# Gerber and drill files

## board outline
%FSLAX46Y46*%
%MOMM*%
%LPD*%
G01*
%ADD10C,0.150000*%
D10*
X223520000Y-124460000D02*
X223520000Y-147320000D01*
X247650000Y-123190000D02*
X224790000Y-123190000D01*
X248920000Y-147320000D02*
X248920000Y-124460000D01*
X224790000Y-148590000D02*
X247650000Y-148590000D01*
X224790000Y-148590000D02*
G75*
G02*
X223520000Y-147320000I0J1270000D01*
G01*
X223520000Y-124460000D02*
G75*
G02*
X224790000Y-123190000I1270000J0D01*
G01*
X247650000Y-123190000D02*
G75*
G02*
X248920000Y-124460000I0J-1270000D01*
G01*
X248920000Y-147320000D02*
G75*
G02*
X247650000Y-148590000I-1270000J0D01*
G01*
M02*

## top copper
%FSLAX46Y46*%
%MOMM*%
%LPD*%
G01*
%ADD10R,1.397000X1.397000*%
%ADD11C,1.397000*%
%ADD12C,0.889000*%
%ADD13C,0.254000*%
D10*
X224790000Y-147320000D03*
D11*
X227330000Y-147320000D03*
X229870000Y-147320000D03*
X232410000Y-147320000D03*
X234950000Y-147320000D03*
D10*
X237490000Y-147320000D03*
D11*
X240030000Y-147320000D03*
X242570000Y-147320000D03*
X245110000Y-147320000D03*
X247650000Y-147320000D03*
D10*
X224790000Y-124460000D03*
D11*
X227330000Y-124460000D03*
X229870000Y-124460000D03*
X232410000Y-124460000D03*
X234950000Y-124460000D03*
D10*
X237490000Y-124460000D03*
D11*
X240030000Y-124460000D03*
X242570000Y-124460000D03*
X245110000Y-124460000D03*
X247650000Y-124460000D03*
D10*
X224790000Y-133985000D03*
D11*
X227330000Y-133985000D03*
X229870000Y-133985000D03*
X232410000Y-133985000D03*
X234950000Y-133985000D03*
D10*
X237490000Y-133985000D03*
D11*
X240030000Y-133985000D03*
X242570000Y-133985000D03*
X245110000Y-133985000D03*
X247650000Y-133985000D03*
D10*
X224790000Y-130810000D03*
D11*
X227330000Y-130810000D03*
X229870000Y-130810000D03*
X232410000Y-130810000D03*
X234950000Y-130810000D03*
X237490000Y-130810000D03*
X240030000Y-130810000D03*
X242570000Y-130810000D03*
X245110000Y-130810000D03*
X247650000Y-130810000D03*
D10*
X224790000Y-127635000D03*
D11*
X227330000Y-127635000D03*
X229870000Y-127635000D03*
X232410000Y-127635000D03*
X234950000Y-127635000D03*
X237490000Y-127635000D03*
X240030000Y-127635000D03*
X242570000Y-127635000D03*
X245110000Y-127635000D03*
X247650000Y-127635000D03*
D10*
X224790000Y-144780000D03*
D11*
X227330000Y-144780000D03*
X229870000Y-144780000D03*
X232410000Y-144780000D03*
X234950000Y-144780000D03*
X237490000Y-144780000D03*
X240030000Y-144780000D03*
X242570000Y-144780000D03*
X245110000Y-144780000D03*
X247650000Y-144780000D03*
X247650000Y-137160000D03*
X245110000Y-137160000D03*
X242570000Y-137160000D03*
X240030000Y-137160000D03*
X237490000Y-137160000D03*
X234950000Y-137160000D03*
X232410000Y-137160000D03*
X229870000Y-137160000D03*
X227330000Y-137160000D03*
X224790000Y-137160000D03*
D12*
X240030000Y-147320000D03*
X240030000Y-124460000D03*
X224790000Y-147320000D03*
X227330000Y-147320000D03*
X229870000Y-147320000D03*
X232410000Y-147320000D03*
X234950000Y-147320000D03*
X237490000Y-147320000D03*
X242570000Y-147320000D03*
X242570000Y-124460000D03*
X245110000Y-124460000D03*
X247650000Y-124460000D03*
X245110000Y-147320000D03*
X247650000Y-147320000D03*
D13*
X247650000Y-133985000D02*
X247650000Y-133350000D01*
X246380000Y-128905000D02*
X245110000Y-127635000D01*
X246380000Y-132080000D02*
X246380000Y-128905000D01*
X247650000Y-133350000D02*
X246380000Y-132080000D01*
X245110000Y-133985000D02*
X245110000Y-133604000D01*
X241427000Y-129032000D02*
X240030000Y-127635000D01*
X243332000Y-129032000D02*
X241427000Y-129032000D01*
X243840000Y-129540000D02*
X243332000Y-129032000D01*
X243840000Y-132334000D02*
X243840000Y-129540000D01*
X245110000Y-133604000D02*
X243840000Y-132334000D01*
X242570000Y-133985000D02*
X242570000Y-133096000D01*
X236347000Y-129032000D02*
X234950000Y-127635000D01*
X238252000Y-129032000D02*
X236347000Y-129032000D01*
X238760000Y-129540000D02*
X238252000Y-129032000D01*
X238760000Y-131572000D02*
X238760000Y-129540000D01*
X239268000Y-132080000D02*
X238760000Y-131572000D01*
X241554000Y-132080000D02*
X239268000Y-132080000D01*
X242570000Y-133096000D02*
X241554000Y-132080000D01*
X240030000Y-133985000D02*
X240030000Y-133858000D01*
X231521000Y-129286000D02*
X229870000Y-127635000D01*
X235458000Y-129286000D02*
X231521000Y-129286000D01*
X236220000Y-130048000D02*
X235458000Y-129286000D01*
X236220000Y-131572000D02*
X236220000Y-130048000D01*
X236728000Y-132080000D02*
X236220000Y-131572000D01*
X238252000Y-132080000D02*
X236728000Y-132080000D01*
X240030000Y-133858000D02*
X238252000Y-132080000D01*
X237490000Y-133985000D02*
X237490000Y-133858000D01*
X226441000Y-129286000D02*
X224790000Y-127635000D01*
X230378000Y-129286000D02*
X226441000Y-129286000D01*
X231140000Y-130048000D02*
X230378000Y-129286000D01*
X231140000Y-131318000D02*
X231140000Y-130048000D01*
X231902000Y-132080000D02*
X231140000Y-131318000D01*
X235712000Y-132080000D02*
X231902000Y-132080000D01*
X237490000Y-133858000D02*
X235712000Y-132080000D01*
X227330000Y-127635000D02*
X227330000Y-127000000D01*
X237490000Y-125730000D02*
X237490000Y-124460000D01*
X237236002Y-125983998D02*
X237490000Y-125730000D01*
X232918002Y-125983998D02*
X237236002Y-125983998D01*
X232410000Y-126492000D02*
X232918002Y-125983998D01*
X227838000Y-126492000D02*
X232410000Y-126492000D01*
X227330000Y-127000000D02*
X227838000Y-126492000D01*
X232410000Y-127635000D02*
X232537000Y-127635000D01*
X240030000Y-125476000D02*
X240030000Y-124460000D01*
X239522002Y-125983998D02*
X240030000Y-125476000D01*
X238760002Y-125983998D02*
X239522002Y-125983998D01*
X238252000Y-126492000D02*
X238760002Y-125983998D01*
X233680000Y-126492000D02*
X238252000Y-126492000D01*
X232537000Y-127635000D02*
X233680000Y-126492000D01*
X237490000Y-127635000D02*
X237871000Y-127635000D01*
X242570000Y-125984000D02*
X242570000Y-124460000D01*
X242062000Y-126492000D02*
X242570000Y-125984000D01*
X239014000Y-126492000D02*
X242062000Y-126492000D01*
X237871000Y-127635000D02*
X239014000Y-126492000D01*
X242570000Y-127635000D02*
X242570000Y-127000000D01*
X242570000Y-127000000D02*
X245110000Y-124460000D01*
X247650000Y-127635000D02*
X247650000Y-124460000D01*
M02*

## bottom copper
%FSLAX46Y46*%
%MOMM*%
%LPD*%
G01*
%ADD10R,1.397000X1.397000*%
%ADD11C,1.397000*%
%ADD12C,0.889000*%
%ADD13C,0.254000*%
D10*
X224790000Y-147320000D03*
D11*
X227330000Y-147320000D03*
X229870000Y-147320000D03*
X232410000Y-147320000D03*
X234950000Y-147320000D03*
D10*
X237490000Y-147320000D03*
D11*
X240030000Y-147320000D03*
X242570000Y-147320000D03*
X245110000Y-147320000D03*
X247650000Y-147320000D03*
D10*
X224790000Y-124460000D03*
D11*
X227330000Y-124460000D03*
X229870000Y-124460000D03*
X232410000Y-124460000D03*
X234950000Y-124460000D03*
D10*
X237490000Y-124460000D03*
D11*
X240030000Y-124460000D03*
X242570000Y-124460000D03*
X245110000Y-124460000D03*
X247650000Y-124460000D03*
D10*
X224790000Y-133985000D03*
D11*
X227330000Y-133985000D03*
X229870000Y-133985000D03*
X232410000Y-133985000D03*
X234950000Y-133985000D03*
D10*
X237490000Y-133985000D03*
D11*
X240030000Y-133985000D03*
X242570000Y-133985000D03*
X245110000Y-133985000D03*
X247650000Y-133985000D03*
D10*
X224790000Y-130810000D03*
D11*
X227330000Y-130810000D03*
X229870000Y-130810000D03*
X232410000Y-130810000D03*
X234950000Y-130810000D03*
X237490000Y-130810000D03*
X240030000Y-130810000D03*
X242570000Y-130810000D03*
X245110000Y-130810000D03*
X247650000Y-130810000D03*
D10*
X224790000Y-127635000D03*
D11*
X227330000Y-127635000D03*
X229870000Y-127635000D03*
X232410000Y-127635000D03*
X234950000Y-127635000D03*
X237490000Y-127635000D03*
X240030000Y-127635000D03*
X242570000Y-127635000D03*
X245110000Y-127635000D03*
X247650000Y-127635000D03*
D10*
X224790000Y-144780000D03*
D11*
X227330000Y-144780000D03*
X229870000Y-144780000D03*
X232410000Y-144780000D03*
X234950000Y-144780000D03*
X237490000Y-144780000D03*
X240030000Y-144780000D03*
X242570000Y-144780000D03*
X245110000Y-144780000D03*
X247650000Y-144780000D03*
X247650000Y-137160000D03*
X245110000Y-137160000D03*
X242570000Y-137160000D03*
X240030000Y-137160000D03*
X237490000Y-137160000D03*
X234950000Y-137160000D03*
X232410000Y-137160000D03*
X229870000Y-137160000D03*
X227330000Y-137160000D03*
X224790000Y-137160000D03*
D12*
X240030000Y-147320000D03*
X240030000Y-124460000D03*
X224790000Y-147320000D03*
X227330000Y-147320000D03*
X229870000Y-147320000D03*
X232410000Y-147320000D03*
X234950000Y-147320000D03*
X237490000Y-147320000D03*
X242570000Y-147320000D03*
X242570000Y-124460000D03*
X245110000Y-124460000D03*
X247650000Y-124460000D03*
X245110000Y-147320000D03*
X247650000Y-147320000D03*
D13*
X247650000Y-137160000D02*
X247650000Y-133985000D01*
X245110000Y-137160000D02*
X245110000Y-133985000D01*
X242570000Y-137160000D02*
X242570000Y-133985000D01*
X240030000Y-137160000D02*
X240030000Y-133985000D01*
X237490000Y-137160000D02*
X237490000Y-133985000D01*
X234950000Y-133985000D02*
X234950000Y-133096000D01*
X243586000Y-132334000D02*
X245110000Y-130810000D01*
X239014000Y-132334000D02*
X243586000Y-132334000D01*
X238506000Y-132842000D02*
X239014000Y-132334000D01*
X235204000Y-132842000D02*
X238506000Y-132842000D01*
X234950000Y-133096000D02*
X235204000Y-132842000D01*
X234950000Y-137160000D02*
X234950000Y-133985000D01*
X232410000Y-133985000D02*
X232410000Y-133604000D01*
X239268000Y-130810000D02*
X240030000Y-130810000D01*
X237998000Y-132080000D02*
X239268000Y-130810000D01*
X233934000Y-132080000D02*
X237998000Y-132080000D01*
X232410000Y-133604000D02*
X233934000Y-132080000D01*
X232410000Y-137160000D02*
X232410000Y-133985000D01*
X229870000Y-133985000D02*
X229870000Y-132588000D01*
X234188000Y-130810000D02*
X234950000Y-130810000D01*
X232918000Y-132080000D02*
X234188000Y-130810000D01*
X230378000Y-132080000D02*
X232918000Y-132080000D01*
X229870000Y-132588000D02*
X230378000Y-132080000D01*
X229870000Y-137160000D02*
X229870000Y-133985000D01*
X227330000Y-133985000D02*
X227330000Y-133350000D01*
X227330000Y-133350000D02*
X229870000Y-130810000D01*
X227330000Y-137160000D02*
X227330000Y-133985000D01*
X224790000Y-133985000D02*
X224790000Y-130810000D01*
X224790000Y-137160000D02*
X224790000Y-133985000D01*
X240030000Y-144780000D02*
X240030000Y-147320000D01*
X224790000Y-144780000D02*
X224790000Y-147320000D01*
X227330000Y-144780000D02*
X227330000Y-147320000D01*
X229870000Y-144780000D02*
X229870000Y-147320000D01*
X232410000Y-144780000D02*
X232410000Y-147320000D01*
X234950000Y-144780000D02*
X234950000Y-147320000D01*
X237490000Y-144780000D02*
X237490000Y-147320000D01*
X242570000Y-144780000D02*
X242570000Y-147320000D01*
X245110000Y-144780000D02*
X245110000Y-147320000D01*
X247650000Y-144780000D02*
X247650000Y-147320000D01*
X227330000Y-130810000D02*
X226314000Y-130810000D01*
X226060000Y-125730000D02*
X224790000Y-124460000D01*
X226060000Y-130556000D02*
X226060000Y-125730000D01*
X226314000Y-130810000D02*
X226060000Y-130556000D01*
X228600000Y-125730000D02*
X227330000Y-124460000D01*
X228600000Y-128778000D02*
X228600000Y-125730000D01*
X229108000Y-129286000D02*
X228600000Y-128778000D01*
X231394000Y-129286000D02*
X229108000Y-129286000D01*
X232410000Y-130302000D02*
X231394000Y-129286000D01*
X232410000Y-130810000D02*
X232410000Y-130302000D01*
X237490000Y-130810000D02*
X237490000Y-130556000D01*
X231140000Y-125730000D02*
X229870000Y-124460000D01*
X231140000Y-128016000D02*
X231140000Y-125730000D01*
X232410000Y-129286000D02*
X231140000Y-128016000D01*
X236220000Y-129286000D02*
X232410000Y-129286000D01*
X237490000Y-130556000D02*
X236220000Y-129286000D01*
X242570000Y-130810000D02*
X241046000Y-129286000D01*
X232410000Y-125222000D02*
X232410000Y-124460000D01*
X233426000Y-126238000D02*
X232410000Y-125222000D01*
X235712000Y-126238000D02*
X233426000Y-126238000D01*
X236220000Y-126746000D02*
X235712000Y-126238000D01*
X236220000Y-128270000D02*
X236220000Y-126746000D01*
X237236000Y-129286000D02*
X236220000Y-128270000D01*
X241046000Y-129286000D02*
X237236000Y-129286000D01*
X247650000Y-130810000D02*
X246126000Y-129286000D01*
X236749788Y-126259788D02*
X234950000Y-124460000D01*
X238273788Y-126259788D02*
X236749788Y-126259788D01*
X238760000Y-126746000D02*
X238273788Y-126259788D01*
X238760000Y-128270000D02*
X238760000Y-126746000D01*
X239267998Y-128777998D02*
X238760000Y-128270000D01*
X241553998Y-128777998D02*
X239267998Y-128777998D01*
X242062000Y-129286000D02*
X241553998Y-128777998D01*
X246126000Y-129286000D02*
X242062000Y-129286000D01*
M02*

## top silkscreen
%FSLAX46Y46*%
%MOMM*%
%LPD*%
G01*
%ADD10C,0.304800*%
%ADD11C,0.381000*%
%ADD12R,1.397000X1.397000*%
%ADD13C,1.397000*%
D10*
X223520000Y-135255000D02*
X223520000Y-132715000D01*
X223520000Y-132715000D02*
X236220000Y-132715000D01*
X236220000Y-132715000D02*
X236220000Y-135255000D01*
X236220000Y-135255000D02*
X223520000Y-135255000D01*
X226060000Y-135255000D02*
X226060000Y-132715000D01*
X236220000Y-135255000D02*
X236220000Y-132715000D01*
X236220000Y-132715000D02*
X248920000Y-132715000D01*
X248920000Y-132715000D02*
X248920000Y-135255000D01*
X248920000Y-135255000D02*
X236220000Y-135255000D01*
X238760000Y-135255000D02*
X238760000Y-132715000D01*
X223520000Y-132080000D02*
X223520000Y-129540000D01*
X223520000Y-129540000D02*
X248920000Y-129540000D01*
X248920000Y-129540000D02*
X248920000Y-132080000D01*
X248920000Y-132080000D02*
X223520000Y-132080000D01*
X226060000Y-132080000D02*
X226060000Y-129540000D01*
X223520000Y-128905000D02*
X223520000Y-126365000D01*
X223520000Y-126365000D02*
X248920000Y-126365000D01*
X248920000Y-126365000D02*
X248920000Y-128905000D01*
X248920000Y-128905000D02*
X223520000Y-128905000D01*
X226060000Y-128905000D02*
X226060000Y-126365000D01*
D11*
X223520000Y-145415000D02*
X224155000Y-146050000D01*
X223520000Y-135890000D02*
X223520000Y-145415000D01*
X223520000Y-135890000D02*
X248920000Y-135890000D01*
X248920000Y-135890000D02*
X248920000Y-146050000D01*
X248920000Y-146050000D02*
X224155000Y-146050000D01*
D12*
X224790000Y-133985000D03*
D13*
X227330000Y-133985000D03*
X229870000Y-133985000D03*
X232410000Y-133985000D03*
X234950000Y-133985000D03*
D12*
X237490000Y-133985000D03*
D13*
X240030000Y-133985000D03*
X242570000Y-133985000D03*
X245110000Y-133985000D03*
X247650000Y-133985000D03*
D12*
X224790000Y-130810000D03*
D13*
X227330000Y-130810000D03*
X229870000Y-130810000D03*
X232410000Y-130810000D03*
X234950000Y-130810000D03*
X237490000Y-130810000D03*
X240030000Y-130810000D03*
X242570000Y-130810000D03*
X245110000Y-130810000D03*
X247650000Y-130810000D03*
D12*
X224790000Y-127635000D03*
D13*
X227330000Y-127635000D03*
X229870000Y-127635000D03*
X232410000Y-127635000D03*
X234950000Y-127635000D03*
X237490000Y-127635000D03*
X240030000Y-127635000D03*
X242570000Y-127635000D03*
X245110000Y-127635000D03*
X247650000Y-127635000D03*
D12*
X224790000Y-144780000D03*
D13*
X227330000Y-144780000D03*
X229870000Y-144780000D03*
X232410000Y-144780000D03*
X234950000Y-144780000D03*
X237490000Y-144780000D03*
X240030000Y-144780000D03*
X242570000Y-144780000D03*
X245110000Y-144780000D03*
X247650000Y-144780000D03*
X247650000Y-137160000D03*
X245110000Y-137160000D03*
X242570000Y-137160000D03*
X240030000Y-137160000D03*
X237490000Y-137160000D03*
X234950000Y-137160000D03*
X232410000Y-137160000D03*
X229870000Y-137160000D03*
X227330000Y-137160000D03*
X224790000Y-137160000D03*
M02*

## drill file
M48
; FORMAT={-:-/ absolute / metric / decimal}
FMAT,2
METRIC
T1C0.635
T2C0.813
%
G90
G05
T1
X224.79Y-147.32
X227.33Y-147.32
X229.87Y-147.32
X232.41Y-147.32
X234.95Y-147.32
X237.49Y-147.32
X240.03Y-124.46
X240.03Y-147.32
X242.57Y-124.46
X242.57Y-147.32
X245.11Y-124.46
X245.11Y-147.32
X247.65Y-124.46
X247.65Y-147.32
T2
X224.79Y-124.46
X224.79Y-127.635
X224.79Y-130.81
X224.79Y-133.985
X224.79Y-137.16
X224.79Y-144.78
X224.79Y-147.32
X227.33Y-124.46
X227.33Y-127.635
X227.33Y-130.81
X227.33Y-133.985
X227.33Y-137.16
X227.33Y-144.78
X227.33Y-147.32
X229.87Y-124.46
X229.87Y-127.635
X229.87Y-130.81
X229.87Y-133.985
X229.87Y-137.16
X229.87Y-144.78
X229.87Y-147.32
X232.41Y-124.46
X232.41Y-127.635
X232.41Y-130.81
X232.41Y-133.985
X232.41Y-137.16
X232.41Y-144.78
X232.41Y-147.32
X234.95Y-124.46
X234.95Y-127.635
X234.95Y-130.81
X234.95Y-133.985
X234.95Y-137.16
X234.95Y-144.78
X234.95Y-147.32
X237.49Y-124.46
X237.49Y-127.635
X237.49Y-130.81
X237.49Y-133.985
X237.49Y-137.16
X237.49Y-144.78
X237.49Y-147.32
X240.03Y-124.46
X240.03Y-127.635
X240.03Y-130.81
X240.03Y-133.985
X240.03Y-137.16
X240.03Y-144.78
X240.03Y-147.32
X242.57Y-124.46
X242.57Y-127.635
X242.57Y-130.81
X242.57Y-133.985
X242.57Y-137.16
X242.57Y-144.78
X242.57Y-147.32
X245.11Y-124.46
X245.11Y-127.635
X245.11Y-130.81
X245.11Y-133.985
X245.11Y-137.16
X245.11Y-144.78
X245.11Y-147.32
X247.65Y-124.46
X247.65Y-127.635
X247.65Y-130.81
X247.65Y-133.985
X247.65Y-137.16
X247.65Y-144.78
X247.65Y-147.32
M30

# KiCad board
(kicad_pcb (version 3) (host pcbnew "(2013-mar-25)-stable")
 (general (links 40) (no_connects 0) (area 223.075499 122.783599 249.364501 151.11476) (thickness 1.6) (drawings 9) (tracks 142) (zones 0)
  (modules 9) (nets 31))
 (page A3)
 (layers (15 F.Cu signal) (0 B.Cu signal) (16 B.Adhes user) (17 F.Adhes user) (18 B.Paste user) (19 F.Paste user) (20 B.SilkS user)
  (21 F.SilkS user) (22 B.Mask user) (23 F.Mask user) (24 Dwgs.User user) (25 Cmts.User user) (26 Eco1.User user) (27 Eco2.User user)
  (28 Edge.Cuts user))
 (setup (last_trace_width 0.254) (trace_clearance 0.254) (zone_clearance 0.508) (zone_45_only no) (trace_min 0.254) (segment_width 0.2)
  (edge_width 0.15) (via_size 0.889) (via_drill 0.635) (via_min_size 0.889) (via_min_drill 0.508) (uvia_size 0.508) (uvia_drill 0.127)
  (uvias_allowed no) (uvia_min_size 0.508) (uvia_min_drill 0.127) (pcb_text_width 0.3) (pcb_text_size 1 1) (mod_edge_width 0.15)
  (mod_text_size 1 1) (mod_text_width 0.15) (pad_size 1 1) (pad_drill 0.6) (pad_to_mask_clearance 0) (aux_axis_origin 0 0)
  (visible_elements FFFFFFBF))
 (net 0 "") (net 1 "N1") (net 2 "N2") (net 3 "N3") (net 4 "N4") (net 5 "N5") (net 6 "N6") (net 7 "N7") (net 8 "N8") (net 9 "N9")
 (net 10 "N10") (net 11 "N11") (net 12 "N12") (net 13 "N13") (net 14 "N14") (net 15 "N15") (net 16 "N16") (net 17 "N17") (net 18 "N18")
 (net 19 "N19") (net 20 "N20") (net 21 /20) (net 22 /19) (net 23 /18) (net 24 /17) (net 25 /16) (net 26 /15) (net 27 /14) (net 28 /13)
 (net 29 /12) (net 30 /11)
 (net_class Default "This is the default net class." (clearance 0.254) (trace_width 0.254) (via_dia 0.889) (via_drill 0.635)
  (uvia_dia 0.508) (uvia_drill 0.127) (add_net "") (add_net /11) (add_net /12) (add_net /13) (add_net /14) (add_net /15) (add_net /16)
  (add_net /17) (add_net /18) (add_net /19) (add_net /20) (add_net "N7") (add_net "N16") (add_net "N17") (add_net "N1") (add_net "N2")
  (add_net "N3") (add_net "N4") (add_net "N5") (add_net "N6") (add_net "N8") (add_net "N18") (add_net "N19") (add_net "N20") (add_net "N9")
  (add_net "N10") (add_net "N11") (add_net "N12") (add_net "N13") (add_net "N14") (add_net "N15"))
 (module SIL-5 (layer B.Cu) (at 231.14 147.32)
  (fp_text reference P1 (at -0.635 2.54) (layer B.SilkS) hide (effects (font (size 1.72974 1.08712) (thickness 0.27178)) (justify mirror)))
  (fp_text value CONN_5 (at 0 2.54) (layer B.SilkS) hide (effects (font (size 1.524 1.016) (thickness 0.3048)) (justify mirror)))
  (pad 1 thru_hole rect (at -6.35 0) (size 1.397 1.397) (drill 0.8128) (layers *.Cu *.Mask B.SilkS) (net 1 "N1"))
  (pad 2 thru_hole circle (at -3.81 0) (size 1.397 1.397) (drill 0.8128) (layers *.Cu *.Mask B.SilkS) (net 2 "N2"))
  (pad 3 thru_hole circle (at -1.27 0) (size 1.397 1.397) (drill 0.8128) (layers *.Cu *.Mask B.SilkS) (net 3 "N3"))
  (pad 4 thru_hole circle (at 1.27 0) (size 1.397 1.397) (drill 0.8128) (layers *.Cu *.Mask B.SilkS) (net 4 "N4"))
  (pad 5 thru_hole circle (at 3.81 0) (size 1.397 1.397) (drill 0.8128) (layers *.Cu *.Mask B.SilkS) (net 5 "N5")))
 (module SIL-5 (layer B.Cu) (at 243.84 147.32)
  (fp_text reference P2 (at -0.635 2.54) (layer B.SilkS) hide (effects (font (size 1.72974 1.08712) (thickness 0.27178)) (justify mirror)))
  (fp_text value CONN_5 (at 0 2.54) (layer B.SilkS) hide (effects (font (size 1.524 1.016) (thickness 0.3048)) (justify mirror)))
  (pad 1 thru_hole rect (at -6.35 0) (size 1.397 1.397) (drill 0.8128) (layers *.Cu *.Mask B.SilkS) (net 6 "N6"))
  (pad 2 thru_hole circle (at -3.81 0) (size 1.397 1.397) (drill 0.8128) (layers *.Cu *.Mask B.SilkS) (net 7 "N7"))
  (pad 3 thru_hole circle (at -1.27 0) (size 1.397 1.397) (drill 0.8128) (layers *.Cu *.Mask B.SilkS) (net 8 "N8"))
  (pad 4 thru_hole circle (at 1.27 0) (size 1.397 1.397) (drill 0.8128) (layers *.Cu *.Mask B.SilkS) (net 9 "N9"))
  (pad 5 thru_hole circle (at 3.81 0) (size 1.397 1.397) (drill 0.8128) (layers *.Cu *.Mask B.SilkS) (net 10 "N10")))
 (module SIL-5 (layer B.Cu) (at 231.14 124.46)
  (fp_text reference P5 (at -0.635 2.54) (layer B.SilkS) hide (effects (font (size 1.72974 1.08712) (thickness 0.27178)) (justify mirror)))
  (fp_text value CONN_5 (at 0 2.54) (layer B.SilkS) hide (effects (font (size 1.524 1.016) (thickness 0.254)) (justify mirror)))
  (pad 1 thru_hole rect (at -6.35 0) (size 1.397 1.397) (drill 0.8128) (layers *.Cu *.Mask B.SilkS) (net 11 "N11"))
  (pad 2 thru_hole circle (at -3.81 0) (size 1.397 1.397) (drill 0.8128) (layers *.Cu *.Mask B.SilkS) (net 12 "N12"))
  (pad 3 thru_hole circle (at -1.27 0) (size 1.397 1.397) (drill 0.8128) (layers *.Cu *.Mask B.SilkS) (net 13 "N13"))
  (pad 4 thru_hole circle (at 1.27 0) (size 1.397 1.397) (drill 0.8128) (layers *.Cu *.Mask B.SilkS) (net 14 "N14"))
  (pad 5 thru_hole circle (at 3.81 0) (size 1.397 1.397) (drill 0.8128) (layers *.Cu *.Mask B.SilkS) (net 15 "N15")))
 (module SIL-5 (layer B.Cu) (at 243.84 124.46)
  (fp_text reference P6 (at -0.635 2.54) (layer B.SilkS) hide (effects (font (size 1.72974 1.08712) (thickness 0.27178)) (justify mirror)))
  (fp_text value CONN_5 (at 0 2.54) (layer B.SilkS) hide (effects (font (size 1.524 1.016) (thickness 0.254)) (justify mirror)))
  (pad 1 thru_hole rect (at -6.35 0) (size 1.397 1.397) (drill 0.8128) (layers *.Cu *.Mask B.SilkS) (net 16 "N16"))
  (pad 2 thru_hole circle (at -3.81 0) (size 1.397 1.397) (drill 0.8128) (layers *.Cu *.Mask B.SilkS) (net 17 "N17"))
  (pad 3 thru_hole circle (at -1.27 0) (size 1.397 1.397) (drill 0.8128) (layers *.Cu *.Mask B.SilkS) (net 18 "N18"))
  (pad 4 thru_hole circle (at 1.27 0) (size 1.397 1.397) (drill 0.8128) (layers *.Cu *.Mask B.SilkS) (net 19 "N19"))
  (pad 5 thru_hole circle (at 3.81 0) (size 1.397 1.397) (drill 0.8128) (layers *.Cu *.Mask B.SilkS) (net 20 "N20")))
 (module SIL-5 (layer F.Cu) (at 231.14 133.985)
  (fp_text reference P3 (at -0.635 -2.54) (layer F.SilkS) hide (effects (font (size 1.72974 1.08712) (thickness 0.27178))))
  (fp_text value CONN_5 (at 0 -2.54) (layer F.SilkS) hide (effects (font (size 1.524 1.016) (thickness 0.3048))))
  (fp_line (start -7.62 1.27) (end -7.62 -1.27) (layer F.SilkS) (width 0.3048))
  (fp_line (start -7.62 -1.27) (end 5.08 -1.27) (layer F.SilkS) (width 0.3048))
  (fp_line (start 5.08 -1.27) (end 5.08 1.27) (layer F.SilkS) (width 0.3048))
  (fp_line (start 5.08 1.27) (end -7.62 1.27) (layer F.SilkS) (width 0.3048))
  (fp_line (start -5.08 1.27) (end -5.08 -1.27) (layer F.SilkS) (width 0.3048))
  (pad 1 thru_hole rect (at -6.35 0) (size 1.397 1.397) (drill 0.8128) (layers *.Cu *.Mask F.SilkS) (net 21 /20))
  (pad 2 thru_hole circle (at -3.81 0) (size 1.397 1.397) (drill 0.8128) (layers *.Cu *.Mask F.SilkS) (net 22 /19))
  (pad 3 thru_hole circle (at -1.27 0) (size 1.397 1.397) (drill 0.8128) (layers *.Cu *.Mask F.SilkS) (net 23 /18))
  (pad 4 thru_hole circle (at 1.27 0) (size 1.397 1.397) (drill 0.8128) (layers *.Cu *.Mask F.SilkS) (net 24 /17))
  (pad 5 thru_hole circle (at 3.81 0) (size 1.397 1.397) (drill 0.8128) (layers *.Cu *.Mask F.SilkS) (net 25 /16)))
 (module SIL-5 (layer F.Cu) (at 243.84 133.985)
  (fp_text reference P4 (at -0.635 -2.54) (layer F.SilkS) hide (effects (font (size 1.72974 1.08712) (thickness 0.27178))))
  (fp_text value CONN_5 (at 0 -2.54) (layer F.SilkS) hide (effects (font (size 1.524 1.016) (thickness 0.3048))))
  (fp_line (start -7.62 1.27) (end -7.62 -1.27) (layer F.SilkS) (width 0.3048))
  (fp_line (start -7.62 -1.27) (end 5.08 -1.27) (layer F.SilkS) (width 0.3048))
  (fp_line (start 5.08 -1.27) (end 5.08 1.27) (layer F.SilkS) (width 0.3048))
  (fp_line (start 5.08 1.27) (end -7.62 1.27) (layer F.SilkS) (width 0.3048))
  (fp_line (start -5.08 1.27) (end -5.08 -1.27) (layer F.SilkS) (width 0.3048))
  (pad 1 thru_hole rect (at -6.35 0) (size 1.397 1.397) (drill 0.8128) (layers *.Cu *.Mask F.SilkS) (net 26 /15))
  (pad 2 thru_hole circle (at -3.81 0) (size 1.397 1.397) (drill 0.8128) (layers *.Cu *.Mask F.SilkS) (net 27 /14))
  (pad 3 thru_hole circle (at -1.27 0) (size 1.397 1.397) (drill 0.8128) (layers *.Cu *.Mask F.SilkS) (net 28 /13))
  (pad 4 thru_hole circle (at 1.27 0) (size 1.397 1.397) (drill 0.8128) (layers *.Cu *.Mask F.SilkS) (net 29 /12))
  (pad 5 thru_hole circle (at 3.81 0) (size 1.397 1.397) (drill 0.8128) (layers *.Cu *.Mask F.SilkS) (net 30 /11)))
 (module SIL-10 (layer F.Cu) (at 236.22 130.81)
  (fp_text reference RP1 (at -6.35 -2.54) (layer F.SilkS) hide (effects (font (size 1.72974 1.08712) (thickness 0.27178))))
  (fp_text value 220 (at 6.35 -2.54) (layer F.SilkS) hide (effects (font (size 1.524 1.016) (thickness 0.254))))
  (fp_line (start -12.7 1.27) (end -12.7 -1.27) (layer F.SilkS) (width 0.3048))
  (fp_line (start -12.7 -1.27) (end 12.7 -1.27) (layer F.SilkS) (width 0.3048))
  (fp_line (start 12.7 -1.27) (end 12.7 1.27) (layer F.SilkS) (width 0.3048))
  (fp_line (start 12.7 1.27) (end -12.7 1.27) (layer F.SilkS) (width 0.3048))
  (fp_line (start -10.16 1.27) (end -10.16 -1.27) (layer F.SilkS) (width 0.3048))
  (pad 1 thru_hole rect (at -11.43 0) (size 1.397 1.397) (drill 0.8128) (layers *.Cu *.Mask F.SilkS) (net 21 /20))
  (pad 2 thru_hole circle (at -8.89 0) (size 1.397 1.397) (drill 0.8128) (layers *.Cu *.Mask F.SilkS) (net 11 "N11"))
  (pad 3 thru_hole circle (at -6.35 0) (size 1.397 1.397) (drill 0.8128) (layers *.Cu *.Mask F.SilkS) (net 22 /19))
  (pad 4 thru_hole circle (at -3.81 0) (size 1.397 1.397) (drill 0.8128) (layers *.Cu *.Mask F.SilkS) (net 12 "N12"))
  (pad 5 thru_hole circle (at -1.27 0) (size 1.397 1.397) (drill 0.8128) (layers *.Cu *.Mask F.SilkS) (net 23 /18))
  (pad 6 thru_hole circle (at 1.27 0) (size 1.397 1.397) (drill 0.8128) (layers *.Cu *.Mask F.SilkS) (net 13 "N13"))
  (pad 7 thru_hole circle (at 3.81 0) (size 1.397 1.397) (drill 0.8128) (layers *.Cu *.Mask F.SilkS) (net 24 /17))
  (pad 8 thru_hole circle (at 6.35 0) (size 1.397 1.397) (drill 0.8128) (layers *.Cu *.Mask F.SilkS) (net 14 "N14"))
  (pad 9 thru_hole circle (at 8.89 0) (size 1.397 1.397) (drill 0.8128) (layers *.Cu *.Mask F.SilkS) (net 25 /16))
  (pad 10 thru_hole circle (at 11.43 0) (size 1.397 1.397) (drill 0.8128) (layers *.Cu *.Mask F.SilkS) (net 15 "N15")))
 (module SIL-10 (layer F.Cu) (at 236.22 127.635)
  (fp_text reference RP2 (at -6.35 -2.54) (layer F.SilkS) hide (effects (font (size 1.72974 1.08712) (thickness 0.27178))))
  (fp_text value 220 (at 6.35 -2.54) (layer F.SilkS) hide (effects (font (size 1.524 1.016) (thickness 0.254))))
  (fp_line (start -12.7 1.27) (end -12.7 -1.27) (layer F.SilkS) (width 0.3048))
  (fp_line (start -12.7 -1.27) (end 12.7 -1.27) (layer F.SilkS) (width 0.3048))
  (fp_line (start 12.7 -1.27) (end 12.7 1.27) (layer F.SilkS) (width 0.3048))
  (fp_line (start 12.7 1.27) (end -12.7 1.27) (layer F.SilkS) (width 0.3048))
  (fp_line (start -10.16 1.27) (end -10.16 -1.27) (layer F.SilkS) (width 0.3048))
  (pad 1 thru_hole rect (at -11.43 0) (size 1.397 1.397) (drill 0.8128) (layers *.Cu *.Mask F.SilkS) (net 26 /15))
  (pad 2 thru_hole circle (at -8.89 0) (size 1.397 1.397) (drill 0.8128) (layers *.Cu *.Mask F.SilkS) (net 16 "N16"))
  (pad 3 thru_hole circle (at -6.35 0) (size 1.397 1.397) (drill 0.8128) (layers *.Cu *.Mask F.SilkS) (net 27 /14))
  (pad 4 thru_hole circle (at -3.81 0) (size 1.397 1.397) (drill 0.8128) (layers *.Cu *.Mask F.SilkS) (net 17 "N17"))
  (pad 5 thru_hole circle (at -1.27 0) (size 1.397 1.397) (drill 0.8128) (layers *.Cu *.Mask F.SilkS) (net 28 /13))
  (pad 6 thru_hole circle (at 1.27 0) (size 1.397 1.397) (drill 0.8128) (layers *.Cu *.Mask F.SilkS) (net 18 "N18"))
  (pad 7 thru_hole circle (at 3.81 0) (size 1.397 1.397) (drill 0.8128) (layers *.Cu *.Mask F.SilkS) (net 29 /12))
  (pad 8 thru_hole circle (at 6.35 0) (size 1.397 1.397) (drill 0.8128) (layers *.Cu *.Mask F.SilkS) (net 19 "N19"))
  (pad 9 thru_hole circle (at 8.89 0) (size 1.397 1.397) (drill 0.8128) (layers *.Cu *.Mask F.SilkS) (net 30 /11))
  (pad 10 thru_hole circle (at 11.43 0) (size 1.397 1.397) (drill 0.8128) (layers *.Cu *.Mask F.SilkS) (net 20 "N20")))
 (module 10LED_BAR (layer F.Cu) (at 236.22 140.97)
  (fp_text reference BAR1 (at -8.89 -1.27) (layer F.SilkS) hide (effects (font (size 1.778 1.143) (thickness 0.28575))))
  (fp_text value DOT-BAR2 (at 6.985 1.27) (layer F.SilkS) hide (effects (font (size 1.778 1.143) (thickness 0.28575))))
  (fp_line (start -12.7 4.445) (end -12.065 5.08) (layer F.SilkS) (width 0.381))
  (fp_line (start -12.7 -5.08) (end -12.7 4.445) (layer F.SilkS) (width 0.381))
  (fp_line (start -12.7 -5.08) (end 12.7 -5.08) (layer F.SilkS) (width 0.381))
  (fp_line (start 12.7 -5.08) (end 12.7 5.08) (layer F.SilkS) (width 0.381))
  (fp_line (start 12.7 5.08) (end -12.065 5.08) (layer F.SilkS) (width 0.381))
  (pad 1 thru_hole rect (at -11.43 3.81) (size 1.397 1.397) (drill 0.8128) (layers *.Cu *.Mask F.SilkS) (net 1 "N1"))
  (pad 2 thru_hole circle (at -8.89 3.81) (size 1.397 1.397) (drill 0.8128) (layers *.Cu *.Mask F.SilkS) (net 2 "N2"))
  (pad 3 thru_hole circle (at -6.35 3.81) (size 1.397 1.397) (drill 0.8128) (layers *.Cu *.Mask F.SilkS) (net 3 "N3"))
  (pad 4 thru_hole circle (at -3.81 3.81) (size 1.397 1.397) (drill 0.8128) (layers *.Cu *.Mask F.SilkS) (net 4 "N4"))
  (pad 5 thru_hole circle (at -1.27 3.81) (size 1.397 1.397) (drill 0.8128) (layers *.Cu *.Mask F.SilkS) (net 5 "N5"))
  (pad 6 thru_hole circle (at 1.27 3.81) (size 1.397 1.397) (drill 0.8128) (layers *.Cu *.Mask F.SilkS) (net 6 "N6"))
  (pad 7 thru_hole circle (at 3.81 3.81) (size 1.397 1.397) (drill 0.8128) (layers *.Cu *.Mask F.SilkS) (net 7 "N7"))
  (pad 8 thru_hole circle (at 6.35 3.81) (size 1.397 1.397) (drill 0.8128) (layers *.Cu *.Mask F.SilkS) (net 8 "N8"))
  (pad 9 thru_hole circle (at 8.89 3.81) (size 1.397 1.397) (drill 0.8128) (layers *.Cu *.Mask F.SilkS) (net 9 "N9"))
  (pad 10 thru_hole circle (at 11.43 3.81) (size 1.397 1.397) (drill 0.8128) (layers *.Cu *.Mask F.SilkS) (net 10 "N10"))
  (pad 11 thru_hole circle (at 11.43 -3.81) (size 1.397 1.397) (drill 0.8128) (layers *.Cu *.Mask F.SilkS) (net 30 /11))
  (pad 12 thru_hole circle (at 8.89 -3.81) (size 1.397 1.397) (drill 0.8128) (layers *.Cu *.Mask F.SilkS) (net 29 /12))
  (pad 13 thru_hole circle (at 6.35 -3.81) (size 1.397 1.397) (drill 0.8128) (layers *.Cu *.Mask F.SilkS) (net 28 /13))
  (pad 14 thru_hole circle (at 3.81 -3.81) (size 1.397 1.397) (drill 0.8128) (layers *.Cu *.Mask F.SilkS) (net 27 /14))
  (pad 15 thru_hole circle (at 1.27 -3.81) (size 1.397 1.397) (drill 0.8128) (layers *.Cu *.Mask F.SilkS) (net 26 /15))
  (pad 16 thru_hole circle (at -1.27 -3.81) (size 1.397 1.397) (drill 0.8128) (layers *.Cu *.Mask F.SilkS) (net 25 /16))
  (pad 17 thru_hole circle (at -3.81 -3.81) (size 1.397 1.397) (drill 0.8128) (layers *.Cu *.Mask F.SilkS) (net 24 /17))
  (pad 18 thru_hole circle (at -6.35 -3.81) (size 1.397 1.397) (drill 0.8128) (layers *.Cu *.Mask F.SilkS) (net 23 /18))
  (pad 19 thru_hole circle (at -8.89 -3.81) (size 1.397 1.397) (drill 0.8128) (layers *.Cu *.Mask F.SilkS) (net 22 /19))
  (pad 20 thru_hole circle (at -11.43 -3.81) (size 1.397 1.397) (drill 0.8128) (layers *.Cu *.Mask F.SilkS) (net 21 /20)))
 (gr_line (start 223.52 124.46) (end 223.52 147.32) (angle 90) (layer Edge.Cuts) (width 0.15))
 (gr_line (start 247.65 123.19) (end 224.79 123.19) (angle 90) (layer Edge.Cuts) (width 0.15))
 (gr_line (start 248.92 147.32) (end 248.92 124.46) (angle 90) (layer Edge.Cuts) (width 0.15))
 (gr_line (start 224.79 148.59) (end 247.65 148.59) (angle 90) (layer Edge.Cuts) (width 0.15))
 (gr_arc (start 224.79 147.32) (end 224.79 148.59) (angle 90) (layer Edge.Cuts) (width 0.15))
 (gr_arc (start 224.79 124.46) (end 223.52 124.46) (angle 90) (layer Edge.Cuts) (width 0.15))
 (gr_arc (start 247.65 124.46) (end 247.65 123.19) (angle 90) (layer Edge.Cuts) (width 0.15))
 (gr_arc (start 247.65 147.32) (end 248.92 147.32) (angle 90) (layer Edge.Cuts) (width 0.15))
 (segment (start 247.65 133.985) (end 247.65 133.35) (width 0.254) (layer F.Cu) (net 30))
 (segment (start 246.38 128.905) (end 245.11 127.635) (width 0.254) (layer F.Cu) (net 30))
 (segment (start 246.38 132.08) (end 246.38 128.905) (width 0.254) (layer F.Cu) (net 30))
 (segment (start 247.65 133.35) (end 246.38 132.08) (width 0.254) (layer F.Cu) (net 30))
 (segment (start 247.65 137.16) (end 247.65 133.985) (width 0.254) (layer B.Cu) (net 30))
 (segment (start 245.11 133.985) (end 245.11 133.604) (width 0.254) (layer F.Cu) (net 29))
 (segment (start 241.427 129.032) (end 240.03 127.635) (width 0.254) (layer F.Cu) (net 29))
 (segment (start 243.332 129.032) (end 241.427 129.032) (width 0.254) (layer F.Cu) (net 29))
 (segment (start 243.84 129.54) (end 243.332 129.032) (width 0.254) (layer F.Cu) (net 29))
 (segment (start 243.84 132.334) (end 243.84 129.54) (width 0.254) (layer F.Cu) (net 29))
 (segment (start 245.11 133.604) (end 243.84 132.334) (width 0.254) (layer F.Cu) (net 29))
 (segment (start 245.11 137.16) (end 245.11 133.985) (width 0.254) (layer B.Cu) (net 29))
 (segment (start 242.57 133.985) (end 242.57 133.096) (width 0.254) (layer F.Cu) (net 28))
 (segment (start 236.347 129.032) (end 234.95 127.635) (width 0.254) (layer F.Cu) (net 28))
 (segment (start 238.252 129.032) (end 236.347 129.032) (width 0.254) (layer F.Cu) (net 28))
 (segment (start 238.76 129.54) (end 238.252 129.032) (width 0.254) (layer F.Cu) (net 28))
 (segment (start 238.76 131.572) (end 238.76 129.54) (width 0.254) (layer F.Cu) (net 28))
 (segment (start 239.268 132.08) (end 238.76 131.572) (width 0.254) (layer F.Cu) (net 28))
 (segment (start 241.554 132.08) (end 239.268 132.08) (width 0.254) (layer F.Cu) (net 28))
 (segment (start 242.57 133.096) (end 241.554 132.08) (width 0.254) (layer F.Cu) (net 28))
 (segment (start 242.57 137.16) (end 242.57 133.985) (width 0.254) (layer B.Cu) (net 28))
 (segment (start 240.03 133.985) (end 240.03 133.858) (width 0.254) (layer F.Cu) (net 27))
 (segment (start 231.521 129.286) (end 229.87 127.635) (width 0.254) (layer F.Cu) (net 27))
 (segment (start 235.458 129.286) (end 231.521 129.286) (width 0.254) (layer F.Cu) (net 27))
 (segment (start 236.22 130.048) (end 235.458 129.286) (width 0.254) (layer F.Cu) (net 27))
 (segment (start 236.22 131.572) (end 236.22 130.048) (width 0.254) (layer F.Cu) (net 27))
 (segment (start 236.728 132.08) (end 236.22 131.572) (width 0.254) (layer F.Cu) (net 27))
 (segment (start 238.252 132.08) (end 236.728 132.08) (width 0.254) (layer F.Cu) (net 27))
 (segment (start 240.03 133.858) (end 238.252 132.08) (width 0.254) (layer F.Cu) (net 27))
 (segment (start 240.03 137.16) (end 240.03 133.985) (width 0.254) (layer B.Cu) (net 27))
 (segment (start 237.49 133.985) (end 237.49 133.858) (width 0.254) (layer F.Cu) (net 26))
 (segment (start 226.441 129.286) (end 224.79 127.635) (width 0.254) (layer F.Cu) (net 26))
 (segment (start 230.378 129.286) (end 226.441 129.286) (width 0.254) (layer F.Cu) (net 26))
 (segment (start 231.14 130.048) (end 230.378 129.286) (width 0.254) (layer F.Cu) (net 26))
 (segment (start 231.14 131.318) (end 231.14 130.048) (width 0.254) (layer F.Cu) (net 26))
 (segment (start 231.902 132.08) (end 231.14 131.318) (width 0.254) (layer F.Cu) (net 26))
 (segment (start 235.712 132.08) (end 231.902 132.08) (width 0.254) (layer F.Cu) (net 26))
 (segment (start 237.49 133.858) (end 235.712 132.08) (width 0.254) (layer F.Cu) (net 26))
 (segment (start 237.49 137.16) (end 237.49 133.985) (width 0.254) (layer B.Cu) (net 26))
 (segment (start 234.95 133.985) (end 234.95 133.096) (width 0.254) (layer B.Cu) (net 25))
 (segment (start 243.586 132.334) (end 245.11 130.81) (width 0.254) (layer B.Cu) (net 25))
 (segment (start 239.014 132.334) (end 243.586 132.334) (width 0.254) (layer B.Cu) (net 25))
 (segment (start 238.506 132.842) (end 239.014 132.334) (width 0.254) (layer B.Cu) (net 25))
 (segment (start 235.204 132.842) (end 238.506 132.842) (width 0.254) (layer B.Cu) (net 25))
 (segment (start 234.95 133.096) (end 235.204 132.842) (width 0.254) (layer B.Cu) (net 25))
 (segment (start 234.95 137.16) (end 234.95 133.985) (width 0.254) (layer B.Cu) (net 25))
 (segment (start 232.41 133.985) (end 232.41 133.604) (width 0.254) (layer B.Cu) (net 24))
 (segment (start 239.268 130.81) (end 240.03 130.81) (width 0.254) (layer B.Cu) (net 24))
 (segment (start 237.998 132.08) (end 239.268 130.81) (width 0.254) (layer B.Cu) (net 24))
 (segment (start 233.934 132.08) (end 237.998 132.08) (width 0.254) (layer B.Cu) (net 24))
 (segment (start 232.41 133.604) (end 233.934 132.08) (width 0.254) (layer B.Cu) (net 24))
 (segment (start 232.41 137.16) (end 232.41 133.985) (width 0.254) (layer B.Cu) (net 24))
 (segment (start 229.87 133.985) (end 229.87 132.588) (width 0.254) (layer B.Cu) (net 23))
 (segment (start 234.188 130.81) (end 234.95 130.81) (width 0.254) (layer B.Cu) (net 23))
 (segment (start 232.918 132.08) (end 234.188 130.81) (width 0.254) (layer B.Cu) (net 23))
 (segment (start 230.378 132.08) (end 232.918 132.08) (width 0.254) (layer B.Cu) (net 23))
 (segment (start 229.87 132.588) (end 230.378 132.08) (width 0.254) (layer B.Cu) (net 23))
 (segment (start 229.87 137.16) (end 229.87 133.985) (width 0.254) (layer B.Cu) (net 23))
 (segment (start 227.33 133.985) (end 227.33 133.35) (width 0.254) (layer B.Cu) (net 22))
 (segment (start 227.33 133.35) (end 229.87 130.81) (width 0.254) (layer B.Cu) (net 22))
 (segment (start 227.33 137.16) (end 227.33 133.985) (width 0.254) (layer B.Cu) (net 22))
 (segment (start 224.79 133.985) (end 224.79 130.81) (width 0.254) (layer B.Cu) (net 21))
 (segment (start 224.79 137.16) (end 224.79 133.985) (width 0.254) (layer B.Cu) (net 21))
 (segment (start 240.03 144.78) (end 240.03 147.32) (width 0.254) (layer B.Cu) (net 7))
 (via (at 240.03 147.32) (size 0.889) (layers F.Cu B.Cu) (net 7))
 (segment (start 227.33 127.635) (end 227.33 127) (width 0.254) (layer F.Cu) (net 16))
 (segment (start 237.49 125.73) (end 237.49 124.46) (width 0.254) (layer F.Cu) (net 16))
 (segment (start 237.236002 125.983998) (end 237.49 125.73) (width 0.254) (layer F.Cu) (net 16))
 (segment (start 232.918002 125.983998) (end 237.236002 125.983998) (width 0.254) (layer F.Cu) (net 16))
 (segment (start 232.41 126.492) (end 232.918002 125.983998) (width 0.254) (layer F.Cu) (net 16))
 (segment (start 227.838 126.492) (end 232.41 126.492) (width 0.254) (layer F.Cu) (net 16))
 (segment (start 227.33 127) (end 227.838 126.492) (width 0.254) (layer F.Cu) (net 16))
 (via (at 240.03 124.46) (size 0.889) (layers F.Cu B.Cu) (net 17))
 (segment (start 232.41 127.635) (end 232.537 127.635) (width 0.254) (layer F.Cu) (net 17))
 (segment (start 240.03 125.476) (end 240.03 124.46) (width 0.254) (layer F.Cu) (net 17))
 (segment (start 239.522002 125.983998) (end 240.03 125.476) (width 0.254) (layer F.Cu) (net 17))
 (segment (start 238.760002 125.983998) (end 239.522002 125.983998) (width 0.254) (layer F.Cu) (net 17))
 (segment (start 238.252 126.492) (end 238.760002 125.983998) (width 0.254) (layer F.Cu) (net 17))
 (segment (start 233.68 126.492) (end 238.252 126.492) (width 0.254) (layer F.Cu) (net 17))
 (segment (start 232.537 127.635) (end 233.68 126.492) (width 0.254) (layer F.Cu) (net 17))
 (segment (start 224.79 144.78) (end 224.79 147.32) (width 0.254) (layer B.Cu) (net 1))
 (via (at 224.79 147.32) (size 0.889) (layers F.Cu B.Cu) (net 1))
 (segment (start 227.33 144.78) (end 227.33 147.32) (width 0.254) (layer B.Cu) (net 2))
 (via (at 227.33 147.32) (size 0.889) (layers F.Cu B.Cu) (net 2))
 (segment (start 229.87 144.78) (end 229.87 147.32) (width 0.254) (layer B.Cu) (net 3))
 (via (at 229.87 147.32) (size 0.889) (layers F.Cu B.Cu) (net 3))
 (segment (start 232.41 144.78) (end 232.41 147.32) (width 0.254) (layer B.Cu) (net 4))
 (via (at 232.41 147.32) (size 0.889) (layers F.Cu B.Cu) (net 4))
 (segment (start 234.95 144.78) (end 234.95 147.32) (width 0.254) (layer B.Cu) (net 5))
 (via (at 234.95 147.32) (size 0.889) (layers F.Cu B.Cu) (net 5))
 (segment (start 237.49 144.78) (end 237.49 147.32) (width 0.254) (layer B.Cu) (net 6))
 (via (at 237.49 147.32) (size 0.889) (layers F.Cu B.Cu) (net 6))
 (segment (start 242.57 144.78) (end 242.57 147.32) (width 0.254) (layer B.Cu) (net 8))
 (via (at 242.57 147.32) (size 0.889) (layers F.Cu B.Cu) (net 8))
 (segment (start 237.49 127.635) (end 237.871 127.635) (width 0.254) (layer F.Cu) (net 18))
 (segment (start 242.57 125.984) (end 242.57 124.46) (width 0.254) (layer F.Cu) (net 18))
 (segment (start 242.062 126.492) (end 242.57 125.984) (width 0.254) (layer F.Cu) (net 18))
 (segment (start 239.014 126.492) (end 242.062 126.492) (width 0.254) (layer F.Cu) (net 18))
 (segment (start 237.871 127.635) (end 239.014 126.492) (width 0.254) (layer F.Cu) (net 18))
 (via (at 242.57 124.46) (size 0.889) (layers F.Cu B.Cu) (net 18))
 (segment (start 242.57 127.635) (end 242.57 127) (width 0.254) (layer F.Cu) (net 19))
 (segment (start 242.57 127) (end 245.11 124.46) (width 0.254) (layer F.Cu) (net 19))
 (via (at 245.11 124.46) (size 0.889) (layers F.Cu B.Cu) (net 19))
 (segment (start 247.65 127.635) (end 247.65 124.46) (width 0.254) (layer F.Cu) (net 20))
 (via (at 247.65 124.46) (size 0.889) (layers F.Cu B.Cu) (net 20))
 (segment (start 245.11 144.78) (end 245.11 147.32) (width 0.254) (layer B.Cu) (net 9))
 (via (at 245.11 147.32) (size 0.889) (layers F.Cu B.Cu) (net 9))
 (segment (start 247.65 144.78) (end 247.65 147.32) (width 0.254) (layer B.Cu) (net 10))
 (via (at 247.65 147.32) (size 0.889) (layers F.Cu B.Cu) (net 10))
 (segment (start 227.33 130.81) (end 226.314 130.81) (width 0.254) (layer B.Cu) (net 11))
 (segment (start 226.06 125.73) (end 224.79 124.46) (width 0.254) (layer B.Cu) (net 11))
 (segment (start 226.06 130.556) (end 226.06 125.73) (width 0.254) (layer B.Cu) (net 11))
 (segment (start 226.314 130.81) (end 226.06 130.556) (width 0.254) (layer B.Cu) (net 11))
 (segment (start 228.6 125.73) (end 227.33 124.46) (width 0.254) (layer B.Cu) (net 12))
 (segment (start 228.6 128.778) (end 228.6 125.73) (width 0.254) (layer B.Cu) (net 12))
 (segment (start 229.108 129.286) (end 228.6 128.778) (width 0.254) (layer B.Cu) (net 12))
 (segment (start 231.394 129.286) (end 229.108 129.286) (width 0.254) (layer B.Cu) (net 12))
 (segment (start 232.41 130.302) (end 231.394 129.286) (width 0.254) (layer B.Cu) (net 12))
 (segment (start 232.41 130.81) (end 232.41 130.302) (width 0.254) (layer B.Cu) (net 12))
 (segment (start 237.49 130.81) (end 237.49 130.556) (width 0.254) (layer B.Cu) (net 13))
 (segment (start 231.14 125.73) (end 229.87 124.46) (width 0.254) (layer B.Cu) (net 13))
 (segment (start 231.14 128.016) (end 231.14 125.73) (width 0.254) (layer B.Cu) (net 13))
 (segment (start 232.41 129.286) (end 231.14 128.016) (width 0.254) (layer B.Cu) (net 13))
 (segment (start 236.22 129.286) (end 232.41 129.286) (width 0.254) (layer B.Cu) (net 13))
 (segment (start 237.49 130.556) (end 236.22 129.286) (width 0.254) (layer B.Cu) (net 13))
 (segment (start 242.57 130.81) (end 241.046 129.286) (width 0.254) (layer B.Cu) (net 14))
 (segment (start 232.41 125.222) (end 232.41 124.46) (width 0.254) (layer B.Cu) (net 14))
 (segment (start 233.426 126.238) (end 232.41 125.222) (width 0.254) (layer B.Cu) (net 14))
 (segment (start 235.712 126.238) (end 233.426 126.238) (width 0.254) (layer B.Cu) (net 14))
 (segment (start 236.22 126.746) (end 235.712 126.238) (width 0.254) (layer B.Cu) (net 14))
 (segment (start 236.22 128.27) (end 236.22 126.746) (width 0.254) (layer B.Cu) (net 14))
 (segment (start 237.236 129.286) (end 236.22 128.27) (width 0.254) (layer B.Cu) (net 14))
 (segment (start 241.046 129.286) (end 237.236 129.286) (width 0.254) (layer B.Cu) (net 14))
 (segment (start 247.65 130.81) (end 246.126 129.286) (width 0.254) (layer B.Cu) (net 15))
 (segment (start 236.749788 126.259788) (end 234.95 124.46) (width 0.254) (layer B.Cu) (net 15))
 (segment (start 238.273788 126.259788) (end 236.749788 126.259788) (width 0.254) (layer B.Cu) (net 15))
 (segment (start 238.76 126.746) (end 238.273788 126.259788) (width 0.254) (layer B.Cu) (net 15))
 (segment (start 238.76 128.27) (end 238.76 126.746) (width 0.254) (layer B.Cu) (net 15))
 (segment (start 239.267998 128.777998) (end 238.76 128.27) (width 0.254) (layer B.Cu) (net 15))
 (segment (start 241.553998 128.777998) (end 239.267998 128.777998) (width 0.254) (layer B.Cu) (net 15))
 (segment (start 242.062 129.286) (end 241.553998 128.777998) (width 0.254) (layer B.Cu) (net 15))
 (segment (start 246.126 129.286) (end 242.062 129.286) (width 0.254) (layer B.Cu) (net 15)))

